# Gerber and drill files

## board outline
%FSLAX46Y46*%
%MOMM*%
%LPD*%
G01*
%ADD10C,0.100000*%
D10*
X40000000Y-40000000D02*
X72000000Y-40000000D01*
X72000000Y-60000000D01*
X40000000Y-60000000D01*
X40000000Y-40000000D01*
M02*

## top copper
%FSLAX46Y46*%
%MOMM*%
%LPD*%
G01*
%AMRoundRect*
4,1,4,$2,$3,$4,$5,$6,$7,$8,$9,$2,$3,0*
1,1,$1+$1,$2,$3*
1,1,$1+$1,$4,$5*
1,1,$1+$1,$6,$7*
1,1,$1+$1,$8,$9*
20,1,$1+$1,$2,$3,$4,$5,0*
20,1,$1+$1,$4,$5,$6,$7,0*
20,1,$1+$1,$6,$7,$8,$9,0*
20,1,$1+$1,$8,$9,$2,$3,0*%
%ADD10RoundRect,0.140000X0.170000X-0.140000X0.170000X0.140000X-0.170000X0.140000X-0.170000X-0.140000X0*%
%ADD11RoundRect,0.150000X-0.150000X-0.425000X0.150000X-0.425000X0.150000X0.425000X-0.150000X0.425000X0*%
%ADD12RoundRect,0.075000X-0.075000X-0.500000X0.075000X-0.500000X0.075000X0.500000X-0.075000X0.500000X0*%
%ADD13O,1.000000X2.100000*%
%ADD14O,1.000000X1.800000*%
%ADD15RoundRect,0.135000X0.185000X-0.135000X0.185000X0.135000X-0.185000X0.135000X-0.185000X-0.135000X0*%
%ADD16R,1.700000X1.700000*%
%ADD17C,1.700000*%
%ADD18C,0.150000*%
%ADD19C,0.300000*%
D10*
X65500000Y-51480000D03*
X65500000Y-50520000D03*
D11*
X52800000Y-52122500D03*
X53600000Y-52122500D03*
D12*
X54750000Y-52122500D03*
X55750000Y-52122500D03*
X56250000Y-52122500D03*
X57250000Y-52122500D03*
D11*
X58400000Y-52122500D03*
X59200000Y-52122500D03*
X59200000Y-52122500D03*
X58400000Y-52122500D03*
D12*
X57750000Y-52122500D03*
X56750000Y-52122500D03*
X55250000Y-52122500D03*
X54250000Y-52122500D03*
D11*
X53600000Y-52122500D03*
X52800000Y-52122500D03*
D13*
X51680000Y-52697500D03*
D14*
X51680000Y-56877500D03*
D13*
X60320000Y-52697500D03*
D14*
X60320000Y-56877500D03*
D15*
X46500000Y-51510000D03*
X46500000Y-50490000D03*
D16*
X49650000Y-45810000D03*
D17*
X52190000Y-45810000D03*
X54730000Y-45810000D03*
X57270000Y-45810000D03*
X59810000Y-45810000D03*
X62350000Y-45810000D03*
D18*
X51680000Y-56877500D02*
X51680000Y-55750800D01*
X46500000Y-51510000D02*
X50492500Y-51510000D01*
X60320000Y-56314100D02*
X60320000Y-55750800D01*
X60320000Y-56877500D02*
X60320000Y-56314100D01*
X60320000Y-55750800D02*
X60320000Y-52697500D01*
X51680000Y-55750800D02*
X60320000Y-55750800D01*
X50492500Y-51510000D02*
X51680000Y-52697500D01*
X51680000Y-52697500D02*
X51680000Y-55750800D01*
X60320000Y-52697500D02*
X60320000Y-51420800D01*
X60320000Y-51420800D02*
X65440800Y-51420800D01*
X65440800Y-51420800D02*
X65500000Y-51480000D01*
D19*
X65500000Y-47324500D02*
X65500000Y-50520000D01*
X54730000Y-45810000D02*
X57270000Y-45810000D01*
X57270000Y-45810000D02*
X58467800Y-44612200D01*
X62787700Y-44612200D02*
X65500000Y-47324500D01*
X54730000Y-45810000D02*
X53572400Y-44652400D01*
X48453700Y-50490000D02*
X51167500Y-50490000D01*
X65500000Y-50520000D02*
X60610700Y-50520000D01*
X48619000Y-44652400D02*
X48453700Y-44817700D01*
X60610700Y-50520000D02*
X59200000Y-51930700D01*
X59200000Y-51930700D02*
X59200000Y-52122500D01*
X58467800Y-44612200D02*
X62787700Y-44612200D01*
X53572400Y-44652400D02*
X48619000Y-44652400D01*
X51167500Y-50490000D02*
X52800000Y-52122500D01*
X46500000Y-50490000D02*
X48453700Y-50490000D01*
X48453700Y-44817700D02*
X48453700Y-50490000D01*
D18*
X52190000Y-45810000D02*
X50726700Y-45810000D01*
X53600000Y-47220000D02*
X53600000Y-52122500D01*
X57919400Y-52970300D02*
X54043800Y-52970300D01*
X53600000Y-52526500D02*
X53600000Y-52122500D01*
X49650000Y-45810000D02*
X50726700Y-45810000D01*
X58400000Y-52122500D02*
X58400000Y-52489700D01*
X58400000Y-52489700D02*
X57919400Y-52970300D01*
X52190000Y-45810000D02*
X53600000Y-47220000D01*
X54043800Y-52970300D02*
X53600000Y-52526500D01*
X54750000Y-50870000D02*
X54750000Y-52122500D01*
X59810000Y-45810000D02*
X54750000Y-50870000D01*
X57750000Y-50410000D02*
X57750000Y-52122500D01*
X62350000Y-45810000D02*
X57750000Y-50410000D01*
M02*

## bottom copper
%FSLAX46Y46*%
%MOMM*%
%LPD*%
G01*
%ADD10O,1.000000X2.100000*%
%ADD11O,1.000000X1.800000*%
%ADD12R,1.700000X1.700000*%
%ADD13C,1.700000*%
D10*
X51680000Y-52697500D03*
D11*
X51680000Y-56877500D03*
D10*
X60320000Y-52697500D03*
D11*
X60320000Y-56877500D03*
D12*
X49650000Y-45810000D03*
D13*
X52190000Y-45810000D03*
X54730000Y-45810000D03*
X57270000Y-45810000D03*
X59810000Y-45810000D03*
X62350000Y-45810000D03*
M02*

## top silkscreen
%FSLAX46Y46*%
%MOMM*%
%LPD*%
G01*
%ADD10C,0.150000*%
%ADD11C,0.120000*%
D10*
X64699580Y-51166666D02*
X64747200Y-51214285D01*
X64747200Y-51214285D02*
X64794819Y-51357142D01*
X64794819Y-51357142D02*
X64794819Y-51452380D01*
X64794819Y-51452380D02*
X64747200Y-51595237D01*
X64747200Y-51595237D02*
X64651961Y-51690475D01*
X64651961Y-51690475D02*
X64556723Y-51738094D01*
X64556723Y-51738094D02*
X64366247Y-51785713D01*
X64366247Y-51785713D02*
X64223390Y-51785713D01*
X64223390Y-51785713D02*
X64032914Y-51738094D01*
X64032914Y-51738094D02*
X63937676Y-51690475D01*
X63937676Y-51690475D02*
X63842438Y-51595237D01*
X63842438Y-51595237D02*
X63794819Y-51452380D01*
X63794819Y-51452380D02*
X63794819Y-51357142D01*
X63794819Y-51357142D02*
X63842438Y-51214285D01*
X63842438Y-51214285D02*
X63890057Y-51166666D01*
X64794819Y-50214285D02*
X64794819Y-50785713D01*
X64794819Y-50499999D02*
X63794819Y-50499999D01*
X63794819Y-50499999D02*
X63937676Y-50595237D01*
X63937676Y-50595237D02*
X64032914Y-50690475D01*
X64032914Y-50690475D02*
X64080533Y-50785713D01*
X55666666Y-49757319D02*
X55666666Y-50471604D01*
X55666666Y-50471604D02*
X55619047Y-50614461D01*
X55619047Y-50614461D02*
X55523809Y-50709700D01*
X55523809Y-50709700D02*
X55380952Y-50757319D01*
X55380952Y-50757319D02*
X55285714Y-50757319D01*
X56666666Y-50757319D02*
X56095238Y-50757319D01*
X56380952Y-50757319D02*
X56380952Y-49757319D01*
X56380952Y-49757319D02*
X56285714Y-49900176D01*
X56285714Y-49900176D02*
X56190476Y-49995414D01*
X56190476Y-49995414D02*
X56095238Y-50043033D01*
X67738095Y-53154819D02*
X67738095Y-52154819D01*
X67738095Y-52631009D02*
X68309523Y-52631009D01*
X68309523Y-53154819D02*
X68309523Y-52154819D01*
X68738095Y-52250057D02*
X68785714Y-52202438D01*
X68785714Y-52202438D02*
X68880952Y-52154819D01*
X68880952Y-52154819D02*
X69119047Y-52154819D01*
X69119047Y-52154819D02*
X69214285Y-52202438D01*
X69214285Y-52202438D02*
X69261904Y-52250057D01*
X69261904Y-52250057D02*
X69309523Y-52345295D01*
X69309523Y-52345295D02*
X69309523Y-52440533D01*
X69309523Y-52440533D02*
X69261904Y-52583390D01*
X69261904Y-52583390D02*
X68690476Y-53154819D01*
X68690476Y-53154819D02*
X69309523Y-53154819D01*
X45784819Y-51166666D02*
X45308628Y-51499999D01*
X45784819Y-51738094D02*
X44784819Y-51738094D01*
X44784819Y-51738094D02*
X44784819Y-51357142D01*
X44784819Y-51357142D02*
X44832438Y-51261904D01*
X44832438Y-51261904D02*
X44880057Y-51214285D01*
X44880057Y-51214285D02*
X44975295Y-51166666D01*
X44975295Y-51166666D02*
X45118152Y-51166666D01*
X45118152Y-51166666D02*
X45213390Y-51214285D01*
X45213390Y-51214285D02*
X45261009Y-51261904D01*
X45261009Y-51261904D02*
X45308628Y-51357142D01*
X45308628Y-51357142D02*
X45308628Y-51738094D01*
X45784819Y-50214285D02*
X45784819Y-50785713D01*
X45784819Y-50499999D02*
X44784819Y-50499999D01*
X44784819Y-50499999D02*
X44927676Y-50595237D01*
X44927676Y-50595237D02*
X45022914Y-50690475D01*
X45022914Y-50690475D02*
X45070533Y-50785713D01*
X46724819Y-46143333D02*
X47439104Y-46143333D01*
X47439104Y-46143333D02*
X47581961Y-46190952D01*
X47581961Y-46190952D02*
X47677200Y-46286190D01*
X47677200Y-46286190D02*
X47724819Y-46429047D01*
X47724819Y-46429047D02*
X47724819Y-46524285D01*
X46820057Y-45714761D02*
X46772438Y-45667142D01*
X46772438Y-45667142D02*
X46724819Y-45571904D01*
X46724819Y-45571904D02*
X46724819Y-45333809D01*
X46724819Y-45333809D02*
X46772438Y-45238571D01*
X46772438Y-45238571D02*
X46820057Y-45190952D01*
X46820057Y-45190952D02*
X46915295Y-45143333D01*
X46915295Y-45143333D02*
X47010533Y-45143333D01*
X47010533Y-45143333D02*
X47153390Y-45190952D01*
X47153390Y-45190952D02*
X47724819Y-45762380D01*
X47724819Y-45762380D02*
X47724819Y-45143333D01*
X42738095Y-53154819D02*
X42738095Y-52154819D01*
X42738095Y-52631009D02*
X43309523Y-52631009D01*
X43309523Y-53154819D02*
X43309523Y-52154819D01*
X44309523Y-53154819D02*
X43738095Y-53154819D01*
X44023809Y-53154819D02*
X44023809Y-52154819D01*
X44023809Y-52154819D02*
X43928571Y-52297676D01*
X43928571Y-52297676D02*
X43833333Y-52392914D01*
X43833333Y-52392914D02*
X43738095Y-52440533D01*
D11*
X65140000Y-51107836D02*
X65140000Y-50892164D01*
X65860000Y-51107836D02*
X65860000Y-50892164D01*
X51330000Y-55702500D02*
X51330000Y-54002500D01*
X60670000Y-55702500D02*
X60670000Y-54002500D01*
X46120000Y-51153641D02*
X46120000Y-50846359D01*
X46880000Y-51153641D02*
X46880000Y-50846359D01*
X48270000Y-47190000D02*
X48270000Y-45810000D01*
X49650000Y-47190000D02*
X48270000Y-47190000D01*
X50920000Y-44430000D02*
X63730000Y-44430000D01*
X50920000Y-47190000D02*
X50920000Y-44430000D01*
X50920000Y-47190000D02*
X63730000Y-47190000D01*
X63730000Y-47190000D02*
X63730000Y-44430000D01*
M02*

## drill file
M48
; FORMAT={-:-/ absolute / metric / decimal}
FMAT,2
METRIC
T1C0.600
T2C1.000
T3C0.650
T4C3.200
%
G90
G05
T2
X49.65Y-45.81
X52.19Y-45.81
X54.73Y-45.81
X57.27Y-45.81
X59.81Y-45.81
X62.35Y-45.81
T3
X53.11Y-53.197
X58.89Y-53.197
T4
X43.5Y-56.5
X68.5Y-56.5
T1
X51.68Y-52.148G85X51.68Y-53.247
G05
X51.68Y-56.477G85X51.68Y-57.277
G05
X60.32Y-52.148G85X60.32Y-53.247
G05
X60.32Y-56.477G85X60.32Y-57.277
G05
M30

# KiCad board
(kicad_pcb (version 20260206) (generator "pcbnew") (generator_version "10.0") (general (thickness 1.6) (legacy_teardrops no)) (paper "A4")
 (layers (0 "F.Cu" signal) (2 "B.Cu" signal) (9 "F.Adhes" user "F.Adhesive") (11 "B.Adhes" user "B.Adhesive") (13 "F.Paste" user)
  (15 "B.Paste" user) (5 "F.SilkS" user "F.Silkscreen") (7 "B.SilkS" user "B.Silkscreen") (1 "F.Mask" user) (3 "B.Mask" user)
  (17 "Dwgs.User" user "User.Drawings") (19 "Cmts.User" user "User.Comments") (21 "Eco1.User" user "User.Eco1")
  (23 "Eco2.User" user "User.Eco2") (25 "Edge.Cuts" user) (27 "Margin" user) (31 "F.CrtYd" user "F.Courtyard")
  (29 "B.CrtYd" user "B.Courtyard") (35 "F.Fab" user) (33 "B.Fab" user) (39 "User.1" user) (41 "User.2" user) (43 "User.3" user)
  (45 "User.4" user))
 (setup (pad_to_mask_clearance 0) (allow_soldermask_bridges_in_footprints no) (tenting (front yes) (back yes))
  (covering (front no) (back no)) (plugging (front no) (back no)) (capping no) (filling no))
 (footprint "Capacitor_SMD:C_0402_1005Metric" (layer "F.Cu") (at 65.5 51 90)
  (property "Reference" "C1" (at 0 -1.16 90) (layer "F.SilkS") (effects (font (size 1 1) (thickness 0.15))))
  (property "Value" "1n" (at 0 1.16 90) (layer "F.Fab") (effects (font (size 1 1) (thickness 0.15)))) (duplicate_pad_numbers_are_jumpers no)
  (fp_line (start -0.107836 -0.36) (end 0.107836 -0.36) (stroke (width 0.12) (type solid)) (layer "F.SilkS"))
  (fp_line (start -0.107836 0.36) (end 0.107836 0.36) (stroke (width 0.12) (type solid)) (layer "F.SilkS"))
  (pad "1" smd roundrect (at -0.48 0 90) (size 0.56 0.62) (layers "F.Cu" "F.Mask" "F.Paste") (roundrect_rratio 0.25) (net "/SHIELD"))
  (pad "2" smd roundrect (at 0.48 0 90) (size 0.56 0.62) (layers "F.Cu" "F.Mask" "F.Paste") (roundrect_rratio 0.25) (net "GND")))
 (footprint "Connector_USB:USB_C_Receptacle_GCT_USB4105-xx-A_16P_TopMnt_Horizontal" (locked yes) (layer "F.Cu") (at 56 55.8025)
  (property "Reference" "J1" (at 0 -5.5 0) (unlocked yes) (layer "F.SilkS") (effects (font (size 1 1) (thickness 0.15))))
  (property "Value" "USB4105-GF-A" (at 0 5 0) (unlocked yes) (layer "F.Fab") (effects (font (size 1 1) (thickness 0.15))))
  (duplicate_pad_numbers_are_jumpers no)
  (fp_line (start -4.67 -0.1) (end -4.67 -1.8) (stroke (width 0.12) (type solid)) (layer "F.SilkS"))
  (fp_line (start 4.67 -0.1) (end 4.67 -1.8) (stroke (width 0.12) (type solid)) (layer "F.SilkS"))
  (pad "" np_thru_hole circle (at -2.89 -2.605) (size 0.65 0.65) (drill 0.65) (layers "*.Cu" "*.Mask"))
  (pad "" np_thru_hole circle (at 2.89 -2.605) (size 0.65 0.65) (drill 0.65) (layers "*.Cu" "*.Mask"))
  (pad "A1" smd roundrect (at -3.2 -3.68) (size 0.6 1.15) (layers "F.Cu" "F.Mask" "F.Paste") (roundrect_rratio 0.25) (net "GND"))
  (pad "A4" smd roundrect (at -2.4 -3.68) (size 0.6 1.15) (layers "F.Cu" "F.Mask" "F.Paste") (roundrect_rratio 0.25) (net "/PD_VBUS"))
  (pad "A5" smd roundrect (at -1.25 -3.68) (size 0.3 1.15) (layers "F.Cu" "F.Mask" "F.Paste") (roundrect_rratio 0.25) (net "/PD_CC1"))
  (pad "A6" smd roundrect (at -0.25 -3.68) (size 0.3 1.15) (layers "F.Cu" "F.Mask" "F.Paste") (roundrect_rratio 0.25)
   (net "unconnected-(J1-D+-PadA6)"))
  (pad "A7" smd roundrect (at 0.25 -3.68) (size 0.3 1.15) (layers "F.Cu" "F.Mask" "F.Paste") (roundrect_rratio 0.25)
   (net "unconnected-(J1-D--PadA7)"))
  (pad "A8" smd roundrect (at 1.25 -3.68) (size 0.3 1.15) (layers "F.Cu" "F.Mask" "F.Paste") (roundrect_rratio 0.25)
   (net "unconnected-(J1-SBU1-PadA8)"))
  (pad "A9" smd roundrect (at 2.4 -3.68) (size 0.6 1.15) (layers "F.Cu" "F.Mask" "F.Paste") (roundrect_rratio 0.25) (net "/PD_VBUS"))
  (pad "A12" smd roundrect (at 3.2 -3.68) (size 0.6 1.15) (layers "F.Cu" "F.Mask" "F.Paste") (roundrect_rratio 0.25) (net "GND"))
  (pad "B1" smd roundrect (at 3.2 -3.68) (size 0.6 1.15) (layers "F.Cu" "F.Mask" "F.Paste") (roundrect_rratio 0.25) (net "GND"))
  (pad "B4" smd roundrect (at 2.4 -3.68) (size 0.6 1.15) (layers "F.Cu" "F.Mask" "F.Paste") (roundrect_rratio 0.25) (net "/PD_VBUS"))
  (pad "B5" smd roundrect (at 1.75 -3.68) (size 0.3 1.15) (layers "F.Cu" "F.Mask" "F.Paste") (roundrect_rratio 0.25) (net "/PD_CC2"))
  (pad "B6" smd roundrect (at 0.75 -3.68) (size 0.3 1.15) (layers "F.Cu" "F.Mask" "F.Paste") (roundrect_rratio 0.25)
   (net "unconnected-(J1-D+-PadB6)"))
  (pad "B7" smd roundrect (at -0.75 -3.68) (size 0.3 1.15) (layers "F.Cu" "F.Mask" "F.Paste") (roundrect_rratio 0.25)
   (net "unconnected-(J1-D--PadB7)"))
  (pad "B8" smd roundrect (at -1.75 -3.68) (size 0.3 1.15) (layers "F.Cu" "F.Mask" "F.Paste") (roundrect_rratio 0.25)
   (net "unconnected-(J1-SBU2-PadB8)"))
  (pad "B9" smd roundrect (at -2.4 -3.68) (size 0.6 1.15) (layers "F.Cu" "F.Mask" "F.Paste") (roundrect_rratio 0.25) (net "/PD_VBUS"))
  (pad "B12" smd roundrect (at -3.2 -3.68) (size 0.6 1.15) (layers "F.Cu" "F.Mask" "F.Paste") (roundrect_rratio 0.25) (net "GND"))
  (pad "SH" thru_hole oval (at -4.32 -3.105) (size 1 2.1) (drill oval 0.6 1.7) (layers "*.Cu" "*.Mask" "F.Paste") (remove_unused_layers no)
   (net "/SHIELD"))
  (pad "SH" thru_hole oval (at -4.32 1.075) (size 1 1.8) (drill oval 0.6 1.4) (layers "*.Cu" "*.Mask" "F.Paste") (remove_unused_layers no)
   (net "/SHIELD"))
  (pad "SH" thru_hole oval (at 4.32 -3.105) (size 1 2.1) (drill oval 0.6 1.7) (layers "*.Cu" "*.Mask" "F.Paste") (remove_unused_layers no)
   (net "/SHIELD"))
  (pad "SH" thru_hole oval (at 4.32 1.075) (size 1 1.8) (drill oval 0.6 1.4) (layers "*.Cu" "*.Mask" "F.Paste") (remove_unused_layers no)
   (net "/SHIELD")))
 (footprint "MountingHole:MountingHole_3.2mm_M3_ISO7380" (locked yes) (layer "F.Cu") (at 68.5 56.5)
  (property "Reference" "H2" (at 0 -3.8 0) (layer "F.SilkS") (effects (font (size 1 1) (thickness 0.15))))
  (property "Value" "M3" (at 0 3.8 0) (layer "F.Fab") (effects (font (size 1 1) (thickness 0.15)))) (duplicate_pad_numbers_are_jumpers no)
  (pad "" np_thru_hole circle (at 0 0) (size 3.2 3.2) (drill 3.2) (layers "*.Cu" "*.Mask") (clearance 0.35)))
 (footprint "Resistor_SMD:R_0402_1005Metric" (layer "F.Cu") (at 46.5 51 90)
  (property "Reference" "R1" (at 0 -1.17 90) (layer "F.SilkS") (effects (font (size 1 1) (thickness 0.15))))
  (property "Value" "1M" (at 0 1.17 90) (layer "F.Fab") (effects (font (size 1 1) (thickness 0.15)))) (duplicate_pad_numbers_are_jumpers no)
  (fp_line (start -0.153641 -0.38) (end 0.153641 -0.38) (stroke (width 0.12) (type solid)) (layer "F.SilkS"))
  (fp_line (start -0.153641 0.38) (end 0.153641 0.38) (stroke (width 0.12) (type solid)) (layer "F.SilkS"))
  (pad "1" smd roundrect (at -0.51 0 90) (size 0.54 0.64) (layers "F.Cu" "F.Mask" "F.Paste") (roundrect_rratio 0.25) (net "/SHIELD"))
  (pad "2" smd roundrect (at 0.51 0 90) (size 0.54 0.64) (layers "F.Cu" "F.Mask" "F.Paste") (roundrect_rratio 0.25) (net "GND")))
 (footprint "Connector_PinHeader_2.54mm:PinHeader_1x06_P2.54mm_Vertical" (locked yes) (layer "F.Cu") (at 49.65 45.81 90)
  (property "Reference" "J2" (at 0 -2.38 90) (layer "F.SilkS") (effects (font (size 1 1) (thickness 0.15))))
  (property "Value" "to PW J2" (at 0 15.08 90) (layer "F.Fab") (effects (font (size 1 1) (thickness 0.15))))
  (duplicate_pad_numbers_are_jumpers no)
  (fp_line (start -1.38 -1.38) (end 0 -1.38) (stroke (width 0.12) (type solid)) (layer "F.SilkS"))
  (fp_line (start -1.38 0) (end -1.38 -1.38) (stroke (width 0.12) (type solid)) (layer "F.SilkS"))
  (fp_line (start 1.38 1.27) (end 1.38 14.08) (stroke (width 0.12) (type solid)) (layer "F.SilkS"))
  (fp_line (start -1.38 1.27) (end 1.38 1.27) (stroke (width 0.12) (type solid)) (layer "F.SilkS"))
  (fp_line (start -1.38 1.27) (end -1.38 14.08) (stroke (width 0.12) (type solid)) (layer "F.SilkS"))
  (fp_line (start -1.38 14.08) (end 1.38 14.08) (stroke (width 0.12) (type solid)) (layer "F.SilkS"))
  (pad "1" thru_hole rect (at 0 0 90) (size 1.7 1.7) (drill 1) (layers "*.Cu" "*.Mask") (remove_unused_layers no) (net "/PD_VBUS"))
  (pad "2" thru_hole circle (at 0 2.54 90) (size 1.7 1.7) (drill 1) (layers "*.Cu" "*.Mask") (remove_unused_layers no) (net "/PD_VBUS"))
  (pad "3" thru_hole circle (at 0 5.08 90) (size 1.7 1.7) (drill 1) (layers "*.Cu" "*.Mask") (remove_unused_layers no) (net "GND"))
  (pad "4" thru_hole circle (at 0 7.62 90) (size 1.7 1.7) (drill 1) (layers "*.Cu" "*.Mask") (remove_unused_layers no) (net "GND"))
  (pad "5" thru_hole circle (at 0 10.16 90) (size 1.7 1.7) (drill 1) (layers "*.Cu" "*.Mask") (remove_unused_layers no) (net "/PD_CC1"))
  (pad "6" thru_hole circle (at 0 12.7 90) (size 1.7 1.7) (drill 1) (layers "*.Cu" "*.Mask") (remove_unused_layers no) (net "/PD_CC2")))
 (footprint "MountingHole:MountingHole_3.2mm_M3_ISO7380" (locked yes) (layer "F.Cu") (at 43.5 56.5)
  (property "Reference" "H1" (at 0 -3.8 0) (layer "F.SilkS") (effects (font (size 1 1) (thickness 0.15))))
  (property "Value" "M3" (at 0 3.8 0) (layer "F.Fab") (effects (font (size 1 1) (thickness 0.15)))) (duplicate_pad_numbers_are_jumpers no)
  (pad "" np_thru_hole circle (at 0 0) (size 3.2 3.2) (drill 3.2) (layers "*.Cu" "*.Mask") (clearance 0.35)))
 (gr_rect (start 40 40) (end 72 60) (stroke (width 0.1) (type default)) (fill no) (layer "Edge.Cuts"))
 (segment (start 51.68 56.8775) (end 51.68 55.7508) (width 0.15) (layer "F.Cu") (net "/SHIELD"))
 (segment (start 46.5 51.51) (end 50.4925 51.51) (width 0.15) (layer "F.Cu") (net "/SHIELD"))
 (segment (start 60.32 56.3141) (end 60.32 55.7508) (width 0.15) (layer "F.Cu") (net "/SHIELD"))
 (segment (start 60.32 56.8775) (end 60.32 56.3141) (width 0.15) (layer "F.Cu") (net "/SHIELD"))
 (segment (start 60.32 55.7508) (end 60.32 52.6975) (width 0.15) (layer "F.Cu") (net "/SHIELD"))
 (segment (start 51.68 55.7508) (end 60.32 55.7508) (width 0.15) (layer "F.Cu") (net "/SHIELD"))
 (segment (start 50.4925 51.51) (end 51.68 52.6975) (width 0.15) (layer "F.Cu") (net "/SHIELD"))
 (segment (start 51.68 52.6975) (end 51.68 55.7508) (width 0.15) (layer "F.Cu") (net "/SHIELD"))
 (segment (start 60.32 52.6975) (end 60.32 51.4208) (width 0.15) (layer "F.Cu") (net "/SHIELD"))
 (segment (start 60.32 51.4208) (end 65.4408 51.4208) (width 0.15) (layer "F.Cu") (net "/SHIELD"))
 (segment (start 65.4408 51.4208) (end 65.5 51.48) (width 0.15) (layer "F.Cu") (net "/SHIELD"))
 (segment (start 65.5 47.3245) (end 65.5 50.52) (width 0.3) (layer "F.Cu") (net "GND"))
 (segment (start 54.73 45.81) (end 57.27 45.81) (width 0.3) (layer "F.Cu") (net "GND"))
 (segment (start 57.27 45.81) (end 58.4678 44.6122) (width 0.3) (layer "F.Cu") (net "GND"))
 (segment (start 62.7877 44.6122) (end 65.5 47.3245) (width 0.3) (layer "F.Cu") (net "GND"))
 (segment (start 54.73 45.81) (end 53.5724 44.6524) (width 0.3) (layer "F.Cu") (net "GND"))
 (segment (start 48.4537 50.49) (end 51.1675 50.49) (width 0.3) (layer "F.Cu") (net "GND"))
 (segment (start 65.5 50.52) (end 60.6107 50.52) (width 0.3) (layer "F.Cu") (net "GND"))
 (segment (start 48.619 44.6524) (end 48.4537 44.8177) (width 0.3) (layer "F.Cu") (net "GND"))
 (segment (start 60.6107 50.52) (end 59.2 51.9307) (width 0.3) (layer "F.Cu") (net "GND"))
 (segment (start 59.2 51.9307) (end 59.2 52.1225) (width 0.3) (layer "F.Cu") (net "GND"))
 (segment (start 58.4678 44.6122) (end 62.7877 44.6122) (width 0.3) (layer "F.Cu") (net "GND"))
 (segment (start 53.5724 44.6524) (end 48.619 44.6524) (width 0.3) (layer "F.Cu") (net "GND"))
 (segment (start 51.1675 50.49) (end 52.8 52.1225) (width 0.3) (layer "F.Cu") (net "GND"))
 (segment (start 46.5 50.49) (end 48.4537 50.49) (width 0.3) (layer "F.Cu") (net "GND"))
 (segment (start 48.4537 44.8177) (end 48.4537 50.49) (width 0.3) (layer "F.Cu") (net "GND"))
 (segment (start 52.19 45.81) (end 50.7267 45.81) (width 0.15) (layer "F.Cu") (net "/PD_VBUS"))
 (segment (start 53.6 47.22) (end 53.6 52.1225) (width 0.15) (layer "F.Cu") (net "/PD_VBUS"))
 (segment (start 57.9194 52.9703) (end 54.0438 52.9703) (width 0.15) (layer "F.Cu") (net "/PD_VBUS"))
 (segment (start 53.6 52.5265) (end 53.6 52.1225) (width 0.15) (layer "F.Cu") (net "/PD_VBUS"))
 (segment (start 49.65 45.81) (end 50.7267 45.81) (width 0.15) (layer "F.Cu") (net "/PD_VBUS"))
 (segment (start 58.4 52.1225) (end 58.4 52.4897) (width 0.15) (layer "F.Cu") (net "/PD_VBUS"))
 (segment (start 58.4 52.4897) (end 57.9194 52.9703) (width 0.15) (layer "F.Cu") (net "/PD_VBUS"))
 (segment (start 52.19 45.81) (end 53.6 47.22) (width 0.15) (layer "F.Cu") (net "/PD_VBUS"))
 (segment (start 54.0438 52.9703) (end 53.6 52.5265) (width 0.15) (layer "F.Cu") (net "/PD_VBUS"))
 (segment (start 54.75 50.87) (end 54.75 52.1225) (width 0.15) (layer "F.Cu") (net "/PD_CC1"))
 (segment (start 59.81 45.81) (end 54.75 50.87) (width 0.15) (layer "F.Cu") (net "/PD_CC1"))
 (segment (start 57.75 50.41) (end 57.75 52.1225) (width 0.15) (layer "F.Cu") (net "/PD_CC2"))
 (segment (start 62.35 45.81) (end 57.75 50.41) (width 0.15) (layer "F.Cu") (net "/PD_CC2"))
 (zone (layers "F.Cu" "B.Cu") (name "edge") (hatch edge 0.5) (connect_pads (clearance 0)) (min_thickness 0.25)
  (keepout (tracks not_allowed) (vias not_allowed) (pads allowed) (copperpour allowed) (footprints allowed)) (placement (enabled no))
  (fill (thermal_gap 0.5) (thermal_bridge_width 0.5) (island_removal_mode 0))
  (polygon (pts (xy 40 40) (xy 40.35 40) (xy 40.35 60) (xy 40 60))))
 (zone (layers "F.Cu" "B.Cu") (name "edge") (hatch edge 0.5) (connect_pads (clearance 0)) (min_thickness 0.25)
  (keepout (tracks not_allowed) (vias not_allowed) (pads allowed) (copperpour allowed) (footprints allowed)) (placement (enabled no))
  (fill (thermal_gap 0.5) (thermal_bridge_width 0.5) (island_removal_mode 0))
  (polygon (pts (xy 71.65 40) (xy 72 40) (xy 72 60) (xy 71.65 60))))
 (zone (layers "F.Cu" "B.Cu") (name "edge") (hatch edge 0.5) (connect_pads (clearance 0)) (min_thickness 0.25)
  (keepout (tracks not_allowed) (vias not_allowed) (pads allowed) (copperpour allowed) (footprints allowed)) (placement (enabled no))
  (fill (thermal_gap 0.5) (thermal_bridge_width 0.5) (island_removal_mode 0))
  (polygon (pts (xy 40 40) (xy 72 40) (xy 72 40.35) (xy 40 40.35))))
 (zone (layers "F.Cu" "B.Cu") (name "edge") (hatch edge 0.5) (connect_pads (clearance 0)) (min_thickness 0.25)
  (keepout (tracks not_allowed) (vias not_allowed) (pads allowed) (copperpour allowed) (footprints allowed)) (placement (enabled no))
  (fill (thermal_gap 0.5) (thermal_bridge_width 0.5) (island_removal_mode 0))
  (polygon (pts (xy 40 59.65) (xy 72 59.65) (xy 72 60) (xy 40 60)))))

